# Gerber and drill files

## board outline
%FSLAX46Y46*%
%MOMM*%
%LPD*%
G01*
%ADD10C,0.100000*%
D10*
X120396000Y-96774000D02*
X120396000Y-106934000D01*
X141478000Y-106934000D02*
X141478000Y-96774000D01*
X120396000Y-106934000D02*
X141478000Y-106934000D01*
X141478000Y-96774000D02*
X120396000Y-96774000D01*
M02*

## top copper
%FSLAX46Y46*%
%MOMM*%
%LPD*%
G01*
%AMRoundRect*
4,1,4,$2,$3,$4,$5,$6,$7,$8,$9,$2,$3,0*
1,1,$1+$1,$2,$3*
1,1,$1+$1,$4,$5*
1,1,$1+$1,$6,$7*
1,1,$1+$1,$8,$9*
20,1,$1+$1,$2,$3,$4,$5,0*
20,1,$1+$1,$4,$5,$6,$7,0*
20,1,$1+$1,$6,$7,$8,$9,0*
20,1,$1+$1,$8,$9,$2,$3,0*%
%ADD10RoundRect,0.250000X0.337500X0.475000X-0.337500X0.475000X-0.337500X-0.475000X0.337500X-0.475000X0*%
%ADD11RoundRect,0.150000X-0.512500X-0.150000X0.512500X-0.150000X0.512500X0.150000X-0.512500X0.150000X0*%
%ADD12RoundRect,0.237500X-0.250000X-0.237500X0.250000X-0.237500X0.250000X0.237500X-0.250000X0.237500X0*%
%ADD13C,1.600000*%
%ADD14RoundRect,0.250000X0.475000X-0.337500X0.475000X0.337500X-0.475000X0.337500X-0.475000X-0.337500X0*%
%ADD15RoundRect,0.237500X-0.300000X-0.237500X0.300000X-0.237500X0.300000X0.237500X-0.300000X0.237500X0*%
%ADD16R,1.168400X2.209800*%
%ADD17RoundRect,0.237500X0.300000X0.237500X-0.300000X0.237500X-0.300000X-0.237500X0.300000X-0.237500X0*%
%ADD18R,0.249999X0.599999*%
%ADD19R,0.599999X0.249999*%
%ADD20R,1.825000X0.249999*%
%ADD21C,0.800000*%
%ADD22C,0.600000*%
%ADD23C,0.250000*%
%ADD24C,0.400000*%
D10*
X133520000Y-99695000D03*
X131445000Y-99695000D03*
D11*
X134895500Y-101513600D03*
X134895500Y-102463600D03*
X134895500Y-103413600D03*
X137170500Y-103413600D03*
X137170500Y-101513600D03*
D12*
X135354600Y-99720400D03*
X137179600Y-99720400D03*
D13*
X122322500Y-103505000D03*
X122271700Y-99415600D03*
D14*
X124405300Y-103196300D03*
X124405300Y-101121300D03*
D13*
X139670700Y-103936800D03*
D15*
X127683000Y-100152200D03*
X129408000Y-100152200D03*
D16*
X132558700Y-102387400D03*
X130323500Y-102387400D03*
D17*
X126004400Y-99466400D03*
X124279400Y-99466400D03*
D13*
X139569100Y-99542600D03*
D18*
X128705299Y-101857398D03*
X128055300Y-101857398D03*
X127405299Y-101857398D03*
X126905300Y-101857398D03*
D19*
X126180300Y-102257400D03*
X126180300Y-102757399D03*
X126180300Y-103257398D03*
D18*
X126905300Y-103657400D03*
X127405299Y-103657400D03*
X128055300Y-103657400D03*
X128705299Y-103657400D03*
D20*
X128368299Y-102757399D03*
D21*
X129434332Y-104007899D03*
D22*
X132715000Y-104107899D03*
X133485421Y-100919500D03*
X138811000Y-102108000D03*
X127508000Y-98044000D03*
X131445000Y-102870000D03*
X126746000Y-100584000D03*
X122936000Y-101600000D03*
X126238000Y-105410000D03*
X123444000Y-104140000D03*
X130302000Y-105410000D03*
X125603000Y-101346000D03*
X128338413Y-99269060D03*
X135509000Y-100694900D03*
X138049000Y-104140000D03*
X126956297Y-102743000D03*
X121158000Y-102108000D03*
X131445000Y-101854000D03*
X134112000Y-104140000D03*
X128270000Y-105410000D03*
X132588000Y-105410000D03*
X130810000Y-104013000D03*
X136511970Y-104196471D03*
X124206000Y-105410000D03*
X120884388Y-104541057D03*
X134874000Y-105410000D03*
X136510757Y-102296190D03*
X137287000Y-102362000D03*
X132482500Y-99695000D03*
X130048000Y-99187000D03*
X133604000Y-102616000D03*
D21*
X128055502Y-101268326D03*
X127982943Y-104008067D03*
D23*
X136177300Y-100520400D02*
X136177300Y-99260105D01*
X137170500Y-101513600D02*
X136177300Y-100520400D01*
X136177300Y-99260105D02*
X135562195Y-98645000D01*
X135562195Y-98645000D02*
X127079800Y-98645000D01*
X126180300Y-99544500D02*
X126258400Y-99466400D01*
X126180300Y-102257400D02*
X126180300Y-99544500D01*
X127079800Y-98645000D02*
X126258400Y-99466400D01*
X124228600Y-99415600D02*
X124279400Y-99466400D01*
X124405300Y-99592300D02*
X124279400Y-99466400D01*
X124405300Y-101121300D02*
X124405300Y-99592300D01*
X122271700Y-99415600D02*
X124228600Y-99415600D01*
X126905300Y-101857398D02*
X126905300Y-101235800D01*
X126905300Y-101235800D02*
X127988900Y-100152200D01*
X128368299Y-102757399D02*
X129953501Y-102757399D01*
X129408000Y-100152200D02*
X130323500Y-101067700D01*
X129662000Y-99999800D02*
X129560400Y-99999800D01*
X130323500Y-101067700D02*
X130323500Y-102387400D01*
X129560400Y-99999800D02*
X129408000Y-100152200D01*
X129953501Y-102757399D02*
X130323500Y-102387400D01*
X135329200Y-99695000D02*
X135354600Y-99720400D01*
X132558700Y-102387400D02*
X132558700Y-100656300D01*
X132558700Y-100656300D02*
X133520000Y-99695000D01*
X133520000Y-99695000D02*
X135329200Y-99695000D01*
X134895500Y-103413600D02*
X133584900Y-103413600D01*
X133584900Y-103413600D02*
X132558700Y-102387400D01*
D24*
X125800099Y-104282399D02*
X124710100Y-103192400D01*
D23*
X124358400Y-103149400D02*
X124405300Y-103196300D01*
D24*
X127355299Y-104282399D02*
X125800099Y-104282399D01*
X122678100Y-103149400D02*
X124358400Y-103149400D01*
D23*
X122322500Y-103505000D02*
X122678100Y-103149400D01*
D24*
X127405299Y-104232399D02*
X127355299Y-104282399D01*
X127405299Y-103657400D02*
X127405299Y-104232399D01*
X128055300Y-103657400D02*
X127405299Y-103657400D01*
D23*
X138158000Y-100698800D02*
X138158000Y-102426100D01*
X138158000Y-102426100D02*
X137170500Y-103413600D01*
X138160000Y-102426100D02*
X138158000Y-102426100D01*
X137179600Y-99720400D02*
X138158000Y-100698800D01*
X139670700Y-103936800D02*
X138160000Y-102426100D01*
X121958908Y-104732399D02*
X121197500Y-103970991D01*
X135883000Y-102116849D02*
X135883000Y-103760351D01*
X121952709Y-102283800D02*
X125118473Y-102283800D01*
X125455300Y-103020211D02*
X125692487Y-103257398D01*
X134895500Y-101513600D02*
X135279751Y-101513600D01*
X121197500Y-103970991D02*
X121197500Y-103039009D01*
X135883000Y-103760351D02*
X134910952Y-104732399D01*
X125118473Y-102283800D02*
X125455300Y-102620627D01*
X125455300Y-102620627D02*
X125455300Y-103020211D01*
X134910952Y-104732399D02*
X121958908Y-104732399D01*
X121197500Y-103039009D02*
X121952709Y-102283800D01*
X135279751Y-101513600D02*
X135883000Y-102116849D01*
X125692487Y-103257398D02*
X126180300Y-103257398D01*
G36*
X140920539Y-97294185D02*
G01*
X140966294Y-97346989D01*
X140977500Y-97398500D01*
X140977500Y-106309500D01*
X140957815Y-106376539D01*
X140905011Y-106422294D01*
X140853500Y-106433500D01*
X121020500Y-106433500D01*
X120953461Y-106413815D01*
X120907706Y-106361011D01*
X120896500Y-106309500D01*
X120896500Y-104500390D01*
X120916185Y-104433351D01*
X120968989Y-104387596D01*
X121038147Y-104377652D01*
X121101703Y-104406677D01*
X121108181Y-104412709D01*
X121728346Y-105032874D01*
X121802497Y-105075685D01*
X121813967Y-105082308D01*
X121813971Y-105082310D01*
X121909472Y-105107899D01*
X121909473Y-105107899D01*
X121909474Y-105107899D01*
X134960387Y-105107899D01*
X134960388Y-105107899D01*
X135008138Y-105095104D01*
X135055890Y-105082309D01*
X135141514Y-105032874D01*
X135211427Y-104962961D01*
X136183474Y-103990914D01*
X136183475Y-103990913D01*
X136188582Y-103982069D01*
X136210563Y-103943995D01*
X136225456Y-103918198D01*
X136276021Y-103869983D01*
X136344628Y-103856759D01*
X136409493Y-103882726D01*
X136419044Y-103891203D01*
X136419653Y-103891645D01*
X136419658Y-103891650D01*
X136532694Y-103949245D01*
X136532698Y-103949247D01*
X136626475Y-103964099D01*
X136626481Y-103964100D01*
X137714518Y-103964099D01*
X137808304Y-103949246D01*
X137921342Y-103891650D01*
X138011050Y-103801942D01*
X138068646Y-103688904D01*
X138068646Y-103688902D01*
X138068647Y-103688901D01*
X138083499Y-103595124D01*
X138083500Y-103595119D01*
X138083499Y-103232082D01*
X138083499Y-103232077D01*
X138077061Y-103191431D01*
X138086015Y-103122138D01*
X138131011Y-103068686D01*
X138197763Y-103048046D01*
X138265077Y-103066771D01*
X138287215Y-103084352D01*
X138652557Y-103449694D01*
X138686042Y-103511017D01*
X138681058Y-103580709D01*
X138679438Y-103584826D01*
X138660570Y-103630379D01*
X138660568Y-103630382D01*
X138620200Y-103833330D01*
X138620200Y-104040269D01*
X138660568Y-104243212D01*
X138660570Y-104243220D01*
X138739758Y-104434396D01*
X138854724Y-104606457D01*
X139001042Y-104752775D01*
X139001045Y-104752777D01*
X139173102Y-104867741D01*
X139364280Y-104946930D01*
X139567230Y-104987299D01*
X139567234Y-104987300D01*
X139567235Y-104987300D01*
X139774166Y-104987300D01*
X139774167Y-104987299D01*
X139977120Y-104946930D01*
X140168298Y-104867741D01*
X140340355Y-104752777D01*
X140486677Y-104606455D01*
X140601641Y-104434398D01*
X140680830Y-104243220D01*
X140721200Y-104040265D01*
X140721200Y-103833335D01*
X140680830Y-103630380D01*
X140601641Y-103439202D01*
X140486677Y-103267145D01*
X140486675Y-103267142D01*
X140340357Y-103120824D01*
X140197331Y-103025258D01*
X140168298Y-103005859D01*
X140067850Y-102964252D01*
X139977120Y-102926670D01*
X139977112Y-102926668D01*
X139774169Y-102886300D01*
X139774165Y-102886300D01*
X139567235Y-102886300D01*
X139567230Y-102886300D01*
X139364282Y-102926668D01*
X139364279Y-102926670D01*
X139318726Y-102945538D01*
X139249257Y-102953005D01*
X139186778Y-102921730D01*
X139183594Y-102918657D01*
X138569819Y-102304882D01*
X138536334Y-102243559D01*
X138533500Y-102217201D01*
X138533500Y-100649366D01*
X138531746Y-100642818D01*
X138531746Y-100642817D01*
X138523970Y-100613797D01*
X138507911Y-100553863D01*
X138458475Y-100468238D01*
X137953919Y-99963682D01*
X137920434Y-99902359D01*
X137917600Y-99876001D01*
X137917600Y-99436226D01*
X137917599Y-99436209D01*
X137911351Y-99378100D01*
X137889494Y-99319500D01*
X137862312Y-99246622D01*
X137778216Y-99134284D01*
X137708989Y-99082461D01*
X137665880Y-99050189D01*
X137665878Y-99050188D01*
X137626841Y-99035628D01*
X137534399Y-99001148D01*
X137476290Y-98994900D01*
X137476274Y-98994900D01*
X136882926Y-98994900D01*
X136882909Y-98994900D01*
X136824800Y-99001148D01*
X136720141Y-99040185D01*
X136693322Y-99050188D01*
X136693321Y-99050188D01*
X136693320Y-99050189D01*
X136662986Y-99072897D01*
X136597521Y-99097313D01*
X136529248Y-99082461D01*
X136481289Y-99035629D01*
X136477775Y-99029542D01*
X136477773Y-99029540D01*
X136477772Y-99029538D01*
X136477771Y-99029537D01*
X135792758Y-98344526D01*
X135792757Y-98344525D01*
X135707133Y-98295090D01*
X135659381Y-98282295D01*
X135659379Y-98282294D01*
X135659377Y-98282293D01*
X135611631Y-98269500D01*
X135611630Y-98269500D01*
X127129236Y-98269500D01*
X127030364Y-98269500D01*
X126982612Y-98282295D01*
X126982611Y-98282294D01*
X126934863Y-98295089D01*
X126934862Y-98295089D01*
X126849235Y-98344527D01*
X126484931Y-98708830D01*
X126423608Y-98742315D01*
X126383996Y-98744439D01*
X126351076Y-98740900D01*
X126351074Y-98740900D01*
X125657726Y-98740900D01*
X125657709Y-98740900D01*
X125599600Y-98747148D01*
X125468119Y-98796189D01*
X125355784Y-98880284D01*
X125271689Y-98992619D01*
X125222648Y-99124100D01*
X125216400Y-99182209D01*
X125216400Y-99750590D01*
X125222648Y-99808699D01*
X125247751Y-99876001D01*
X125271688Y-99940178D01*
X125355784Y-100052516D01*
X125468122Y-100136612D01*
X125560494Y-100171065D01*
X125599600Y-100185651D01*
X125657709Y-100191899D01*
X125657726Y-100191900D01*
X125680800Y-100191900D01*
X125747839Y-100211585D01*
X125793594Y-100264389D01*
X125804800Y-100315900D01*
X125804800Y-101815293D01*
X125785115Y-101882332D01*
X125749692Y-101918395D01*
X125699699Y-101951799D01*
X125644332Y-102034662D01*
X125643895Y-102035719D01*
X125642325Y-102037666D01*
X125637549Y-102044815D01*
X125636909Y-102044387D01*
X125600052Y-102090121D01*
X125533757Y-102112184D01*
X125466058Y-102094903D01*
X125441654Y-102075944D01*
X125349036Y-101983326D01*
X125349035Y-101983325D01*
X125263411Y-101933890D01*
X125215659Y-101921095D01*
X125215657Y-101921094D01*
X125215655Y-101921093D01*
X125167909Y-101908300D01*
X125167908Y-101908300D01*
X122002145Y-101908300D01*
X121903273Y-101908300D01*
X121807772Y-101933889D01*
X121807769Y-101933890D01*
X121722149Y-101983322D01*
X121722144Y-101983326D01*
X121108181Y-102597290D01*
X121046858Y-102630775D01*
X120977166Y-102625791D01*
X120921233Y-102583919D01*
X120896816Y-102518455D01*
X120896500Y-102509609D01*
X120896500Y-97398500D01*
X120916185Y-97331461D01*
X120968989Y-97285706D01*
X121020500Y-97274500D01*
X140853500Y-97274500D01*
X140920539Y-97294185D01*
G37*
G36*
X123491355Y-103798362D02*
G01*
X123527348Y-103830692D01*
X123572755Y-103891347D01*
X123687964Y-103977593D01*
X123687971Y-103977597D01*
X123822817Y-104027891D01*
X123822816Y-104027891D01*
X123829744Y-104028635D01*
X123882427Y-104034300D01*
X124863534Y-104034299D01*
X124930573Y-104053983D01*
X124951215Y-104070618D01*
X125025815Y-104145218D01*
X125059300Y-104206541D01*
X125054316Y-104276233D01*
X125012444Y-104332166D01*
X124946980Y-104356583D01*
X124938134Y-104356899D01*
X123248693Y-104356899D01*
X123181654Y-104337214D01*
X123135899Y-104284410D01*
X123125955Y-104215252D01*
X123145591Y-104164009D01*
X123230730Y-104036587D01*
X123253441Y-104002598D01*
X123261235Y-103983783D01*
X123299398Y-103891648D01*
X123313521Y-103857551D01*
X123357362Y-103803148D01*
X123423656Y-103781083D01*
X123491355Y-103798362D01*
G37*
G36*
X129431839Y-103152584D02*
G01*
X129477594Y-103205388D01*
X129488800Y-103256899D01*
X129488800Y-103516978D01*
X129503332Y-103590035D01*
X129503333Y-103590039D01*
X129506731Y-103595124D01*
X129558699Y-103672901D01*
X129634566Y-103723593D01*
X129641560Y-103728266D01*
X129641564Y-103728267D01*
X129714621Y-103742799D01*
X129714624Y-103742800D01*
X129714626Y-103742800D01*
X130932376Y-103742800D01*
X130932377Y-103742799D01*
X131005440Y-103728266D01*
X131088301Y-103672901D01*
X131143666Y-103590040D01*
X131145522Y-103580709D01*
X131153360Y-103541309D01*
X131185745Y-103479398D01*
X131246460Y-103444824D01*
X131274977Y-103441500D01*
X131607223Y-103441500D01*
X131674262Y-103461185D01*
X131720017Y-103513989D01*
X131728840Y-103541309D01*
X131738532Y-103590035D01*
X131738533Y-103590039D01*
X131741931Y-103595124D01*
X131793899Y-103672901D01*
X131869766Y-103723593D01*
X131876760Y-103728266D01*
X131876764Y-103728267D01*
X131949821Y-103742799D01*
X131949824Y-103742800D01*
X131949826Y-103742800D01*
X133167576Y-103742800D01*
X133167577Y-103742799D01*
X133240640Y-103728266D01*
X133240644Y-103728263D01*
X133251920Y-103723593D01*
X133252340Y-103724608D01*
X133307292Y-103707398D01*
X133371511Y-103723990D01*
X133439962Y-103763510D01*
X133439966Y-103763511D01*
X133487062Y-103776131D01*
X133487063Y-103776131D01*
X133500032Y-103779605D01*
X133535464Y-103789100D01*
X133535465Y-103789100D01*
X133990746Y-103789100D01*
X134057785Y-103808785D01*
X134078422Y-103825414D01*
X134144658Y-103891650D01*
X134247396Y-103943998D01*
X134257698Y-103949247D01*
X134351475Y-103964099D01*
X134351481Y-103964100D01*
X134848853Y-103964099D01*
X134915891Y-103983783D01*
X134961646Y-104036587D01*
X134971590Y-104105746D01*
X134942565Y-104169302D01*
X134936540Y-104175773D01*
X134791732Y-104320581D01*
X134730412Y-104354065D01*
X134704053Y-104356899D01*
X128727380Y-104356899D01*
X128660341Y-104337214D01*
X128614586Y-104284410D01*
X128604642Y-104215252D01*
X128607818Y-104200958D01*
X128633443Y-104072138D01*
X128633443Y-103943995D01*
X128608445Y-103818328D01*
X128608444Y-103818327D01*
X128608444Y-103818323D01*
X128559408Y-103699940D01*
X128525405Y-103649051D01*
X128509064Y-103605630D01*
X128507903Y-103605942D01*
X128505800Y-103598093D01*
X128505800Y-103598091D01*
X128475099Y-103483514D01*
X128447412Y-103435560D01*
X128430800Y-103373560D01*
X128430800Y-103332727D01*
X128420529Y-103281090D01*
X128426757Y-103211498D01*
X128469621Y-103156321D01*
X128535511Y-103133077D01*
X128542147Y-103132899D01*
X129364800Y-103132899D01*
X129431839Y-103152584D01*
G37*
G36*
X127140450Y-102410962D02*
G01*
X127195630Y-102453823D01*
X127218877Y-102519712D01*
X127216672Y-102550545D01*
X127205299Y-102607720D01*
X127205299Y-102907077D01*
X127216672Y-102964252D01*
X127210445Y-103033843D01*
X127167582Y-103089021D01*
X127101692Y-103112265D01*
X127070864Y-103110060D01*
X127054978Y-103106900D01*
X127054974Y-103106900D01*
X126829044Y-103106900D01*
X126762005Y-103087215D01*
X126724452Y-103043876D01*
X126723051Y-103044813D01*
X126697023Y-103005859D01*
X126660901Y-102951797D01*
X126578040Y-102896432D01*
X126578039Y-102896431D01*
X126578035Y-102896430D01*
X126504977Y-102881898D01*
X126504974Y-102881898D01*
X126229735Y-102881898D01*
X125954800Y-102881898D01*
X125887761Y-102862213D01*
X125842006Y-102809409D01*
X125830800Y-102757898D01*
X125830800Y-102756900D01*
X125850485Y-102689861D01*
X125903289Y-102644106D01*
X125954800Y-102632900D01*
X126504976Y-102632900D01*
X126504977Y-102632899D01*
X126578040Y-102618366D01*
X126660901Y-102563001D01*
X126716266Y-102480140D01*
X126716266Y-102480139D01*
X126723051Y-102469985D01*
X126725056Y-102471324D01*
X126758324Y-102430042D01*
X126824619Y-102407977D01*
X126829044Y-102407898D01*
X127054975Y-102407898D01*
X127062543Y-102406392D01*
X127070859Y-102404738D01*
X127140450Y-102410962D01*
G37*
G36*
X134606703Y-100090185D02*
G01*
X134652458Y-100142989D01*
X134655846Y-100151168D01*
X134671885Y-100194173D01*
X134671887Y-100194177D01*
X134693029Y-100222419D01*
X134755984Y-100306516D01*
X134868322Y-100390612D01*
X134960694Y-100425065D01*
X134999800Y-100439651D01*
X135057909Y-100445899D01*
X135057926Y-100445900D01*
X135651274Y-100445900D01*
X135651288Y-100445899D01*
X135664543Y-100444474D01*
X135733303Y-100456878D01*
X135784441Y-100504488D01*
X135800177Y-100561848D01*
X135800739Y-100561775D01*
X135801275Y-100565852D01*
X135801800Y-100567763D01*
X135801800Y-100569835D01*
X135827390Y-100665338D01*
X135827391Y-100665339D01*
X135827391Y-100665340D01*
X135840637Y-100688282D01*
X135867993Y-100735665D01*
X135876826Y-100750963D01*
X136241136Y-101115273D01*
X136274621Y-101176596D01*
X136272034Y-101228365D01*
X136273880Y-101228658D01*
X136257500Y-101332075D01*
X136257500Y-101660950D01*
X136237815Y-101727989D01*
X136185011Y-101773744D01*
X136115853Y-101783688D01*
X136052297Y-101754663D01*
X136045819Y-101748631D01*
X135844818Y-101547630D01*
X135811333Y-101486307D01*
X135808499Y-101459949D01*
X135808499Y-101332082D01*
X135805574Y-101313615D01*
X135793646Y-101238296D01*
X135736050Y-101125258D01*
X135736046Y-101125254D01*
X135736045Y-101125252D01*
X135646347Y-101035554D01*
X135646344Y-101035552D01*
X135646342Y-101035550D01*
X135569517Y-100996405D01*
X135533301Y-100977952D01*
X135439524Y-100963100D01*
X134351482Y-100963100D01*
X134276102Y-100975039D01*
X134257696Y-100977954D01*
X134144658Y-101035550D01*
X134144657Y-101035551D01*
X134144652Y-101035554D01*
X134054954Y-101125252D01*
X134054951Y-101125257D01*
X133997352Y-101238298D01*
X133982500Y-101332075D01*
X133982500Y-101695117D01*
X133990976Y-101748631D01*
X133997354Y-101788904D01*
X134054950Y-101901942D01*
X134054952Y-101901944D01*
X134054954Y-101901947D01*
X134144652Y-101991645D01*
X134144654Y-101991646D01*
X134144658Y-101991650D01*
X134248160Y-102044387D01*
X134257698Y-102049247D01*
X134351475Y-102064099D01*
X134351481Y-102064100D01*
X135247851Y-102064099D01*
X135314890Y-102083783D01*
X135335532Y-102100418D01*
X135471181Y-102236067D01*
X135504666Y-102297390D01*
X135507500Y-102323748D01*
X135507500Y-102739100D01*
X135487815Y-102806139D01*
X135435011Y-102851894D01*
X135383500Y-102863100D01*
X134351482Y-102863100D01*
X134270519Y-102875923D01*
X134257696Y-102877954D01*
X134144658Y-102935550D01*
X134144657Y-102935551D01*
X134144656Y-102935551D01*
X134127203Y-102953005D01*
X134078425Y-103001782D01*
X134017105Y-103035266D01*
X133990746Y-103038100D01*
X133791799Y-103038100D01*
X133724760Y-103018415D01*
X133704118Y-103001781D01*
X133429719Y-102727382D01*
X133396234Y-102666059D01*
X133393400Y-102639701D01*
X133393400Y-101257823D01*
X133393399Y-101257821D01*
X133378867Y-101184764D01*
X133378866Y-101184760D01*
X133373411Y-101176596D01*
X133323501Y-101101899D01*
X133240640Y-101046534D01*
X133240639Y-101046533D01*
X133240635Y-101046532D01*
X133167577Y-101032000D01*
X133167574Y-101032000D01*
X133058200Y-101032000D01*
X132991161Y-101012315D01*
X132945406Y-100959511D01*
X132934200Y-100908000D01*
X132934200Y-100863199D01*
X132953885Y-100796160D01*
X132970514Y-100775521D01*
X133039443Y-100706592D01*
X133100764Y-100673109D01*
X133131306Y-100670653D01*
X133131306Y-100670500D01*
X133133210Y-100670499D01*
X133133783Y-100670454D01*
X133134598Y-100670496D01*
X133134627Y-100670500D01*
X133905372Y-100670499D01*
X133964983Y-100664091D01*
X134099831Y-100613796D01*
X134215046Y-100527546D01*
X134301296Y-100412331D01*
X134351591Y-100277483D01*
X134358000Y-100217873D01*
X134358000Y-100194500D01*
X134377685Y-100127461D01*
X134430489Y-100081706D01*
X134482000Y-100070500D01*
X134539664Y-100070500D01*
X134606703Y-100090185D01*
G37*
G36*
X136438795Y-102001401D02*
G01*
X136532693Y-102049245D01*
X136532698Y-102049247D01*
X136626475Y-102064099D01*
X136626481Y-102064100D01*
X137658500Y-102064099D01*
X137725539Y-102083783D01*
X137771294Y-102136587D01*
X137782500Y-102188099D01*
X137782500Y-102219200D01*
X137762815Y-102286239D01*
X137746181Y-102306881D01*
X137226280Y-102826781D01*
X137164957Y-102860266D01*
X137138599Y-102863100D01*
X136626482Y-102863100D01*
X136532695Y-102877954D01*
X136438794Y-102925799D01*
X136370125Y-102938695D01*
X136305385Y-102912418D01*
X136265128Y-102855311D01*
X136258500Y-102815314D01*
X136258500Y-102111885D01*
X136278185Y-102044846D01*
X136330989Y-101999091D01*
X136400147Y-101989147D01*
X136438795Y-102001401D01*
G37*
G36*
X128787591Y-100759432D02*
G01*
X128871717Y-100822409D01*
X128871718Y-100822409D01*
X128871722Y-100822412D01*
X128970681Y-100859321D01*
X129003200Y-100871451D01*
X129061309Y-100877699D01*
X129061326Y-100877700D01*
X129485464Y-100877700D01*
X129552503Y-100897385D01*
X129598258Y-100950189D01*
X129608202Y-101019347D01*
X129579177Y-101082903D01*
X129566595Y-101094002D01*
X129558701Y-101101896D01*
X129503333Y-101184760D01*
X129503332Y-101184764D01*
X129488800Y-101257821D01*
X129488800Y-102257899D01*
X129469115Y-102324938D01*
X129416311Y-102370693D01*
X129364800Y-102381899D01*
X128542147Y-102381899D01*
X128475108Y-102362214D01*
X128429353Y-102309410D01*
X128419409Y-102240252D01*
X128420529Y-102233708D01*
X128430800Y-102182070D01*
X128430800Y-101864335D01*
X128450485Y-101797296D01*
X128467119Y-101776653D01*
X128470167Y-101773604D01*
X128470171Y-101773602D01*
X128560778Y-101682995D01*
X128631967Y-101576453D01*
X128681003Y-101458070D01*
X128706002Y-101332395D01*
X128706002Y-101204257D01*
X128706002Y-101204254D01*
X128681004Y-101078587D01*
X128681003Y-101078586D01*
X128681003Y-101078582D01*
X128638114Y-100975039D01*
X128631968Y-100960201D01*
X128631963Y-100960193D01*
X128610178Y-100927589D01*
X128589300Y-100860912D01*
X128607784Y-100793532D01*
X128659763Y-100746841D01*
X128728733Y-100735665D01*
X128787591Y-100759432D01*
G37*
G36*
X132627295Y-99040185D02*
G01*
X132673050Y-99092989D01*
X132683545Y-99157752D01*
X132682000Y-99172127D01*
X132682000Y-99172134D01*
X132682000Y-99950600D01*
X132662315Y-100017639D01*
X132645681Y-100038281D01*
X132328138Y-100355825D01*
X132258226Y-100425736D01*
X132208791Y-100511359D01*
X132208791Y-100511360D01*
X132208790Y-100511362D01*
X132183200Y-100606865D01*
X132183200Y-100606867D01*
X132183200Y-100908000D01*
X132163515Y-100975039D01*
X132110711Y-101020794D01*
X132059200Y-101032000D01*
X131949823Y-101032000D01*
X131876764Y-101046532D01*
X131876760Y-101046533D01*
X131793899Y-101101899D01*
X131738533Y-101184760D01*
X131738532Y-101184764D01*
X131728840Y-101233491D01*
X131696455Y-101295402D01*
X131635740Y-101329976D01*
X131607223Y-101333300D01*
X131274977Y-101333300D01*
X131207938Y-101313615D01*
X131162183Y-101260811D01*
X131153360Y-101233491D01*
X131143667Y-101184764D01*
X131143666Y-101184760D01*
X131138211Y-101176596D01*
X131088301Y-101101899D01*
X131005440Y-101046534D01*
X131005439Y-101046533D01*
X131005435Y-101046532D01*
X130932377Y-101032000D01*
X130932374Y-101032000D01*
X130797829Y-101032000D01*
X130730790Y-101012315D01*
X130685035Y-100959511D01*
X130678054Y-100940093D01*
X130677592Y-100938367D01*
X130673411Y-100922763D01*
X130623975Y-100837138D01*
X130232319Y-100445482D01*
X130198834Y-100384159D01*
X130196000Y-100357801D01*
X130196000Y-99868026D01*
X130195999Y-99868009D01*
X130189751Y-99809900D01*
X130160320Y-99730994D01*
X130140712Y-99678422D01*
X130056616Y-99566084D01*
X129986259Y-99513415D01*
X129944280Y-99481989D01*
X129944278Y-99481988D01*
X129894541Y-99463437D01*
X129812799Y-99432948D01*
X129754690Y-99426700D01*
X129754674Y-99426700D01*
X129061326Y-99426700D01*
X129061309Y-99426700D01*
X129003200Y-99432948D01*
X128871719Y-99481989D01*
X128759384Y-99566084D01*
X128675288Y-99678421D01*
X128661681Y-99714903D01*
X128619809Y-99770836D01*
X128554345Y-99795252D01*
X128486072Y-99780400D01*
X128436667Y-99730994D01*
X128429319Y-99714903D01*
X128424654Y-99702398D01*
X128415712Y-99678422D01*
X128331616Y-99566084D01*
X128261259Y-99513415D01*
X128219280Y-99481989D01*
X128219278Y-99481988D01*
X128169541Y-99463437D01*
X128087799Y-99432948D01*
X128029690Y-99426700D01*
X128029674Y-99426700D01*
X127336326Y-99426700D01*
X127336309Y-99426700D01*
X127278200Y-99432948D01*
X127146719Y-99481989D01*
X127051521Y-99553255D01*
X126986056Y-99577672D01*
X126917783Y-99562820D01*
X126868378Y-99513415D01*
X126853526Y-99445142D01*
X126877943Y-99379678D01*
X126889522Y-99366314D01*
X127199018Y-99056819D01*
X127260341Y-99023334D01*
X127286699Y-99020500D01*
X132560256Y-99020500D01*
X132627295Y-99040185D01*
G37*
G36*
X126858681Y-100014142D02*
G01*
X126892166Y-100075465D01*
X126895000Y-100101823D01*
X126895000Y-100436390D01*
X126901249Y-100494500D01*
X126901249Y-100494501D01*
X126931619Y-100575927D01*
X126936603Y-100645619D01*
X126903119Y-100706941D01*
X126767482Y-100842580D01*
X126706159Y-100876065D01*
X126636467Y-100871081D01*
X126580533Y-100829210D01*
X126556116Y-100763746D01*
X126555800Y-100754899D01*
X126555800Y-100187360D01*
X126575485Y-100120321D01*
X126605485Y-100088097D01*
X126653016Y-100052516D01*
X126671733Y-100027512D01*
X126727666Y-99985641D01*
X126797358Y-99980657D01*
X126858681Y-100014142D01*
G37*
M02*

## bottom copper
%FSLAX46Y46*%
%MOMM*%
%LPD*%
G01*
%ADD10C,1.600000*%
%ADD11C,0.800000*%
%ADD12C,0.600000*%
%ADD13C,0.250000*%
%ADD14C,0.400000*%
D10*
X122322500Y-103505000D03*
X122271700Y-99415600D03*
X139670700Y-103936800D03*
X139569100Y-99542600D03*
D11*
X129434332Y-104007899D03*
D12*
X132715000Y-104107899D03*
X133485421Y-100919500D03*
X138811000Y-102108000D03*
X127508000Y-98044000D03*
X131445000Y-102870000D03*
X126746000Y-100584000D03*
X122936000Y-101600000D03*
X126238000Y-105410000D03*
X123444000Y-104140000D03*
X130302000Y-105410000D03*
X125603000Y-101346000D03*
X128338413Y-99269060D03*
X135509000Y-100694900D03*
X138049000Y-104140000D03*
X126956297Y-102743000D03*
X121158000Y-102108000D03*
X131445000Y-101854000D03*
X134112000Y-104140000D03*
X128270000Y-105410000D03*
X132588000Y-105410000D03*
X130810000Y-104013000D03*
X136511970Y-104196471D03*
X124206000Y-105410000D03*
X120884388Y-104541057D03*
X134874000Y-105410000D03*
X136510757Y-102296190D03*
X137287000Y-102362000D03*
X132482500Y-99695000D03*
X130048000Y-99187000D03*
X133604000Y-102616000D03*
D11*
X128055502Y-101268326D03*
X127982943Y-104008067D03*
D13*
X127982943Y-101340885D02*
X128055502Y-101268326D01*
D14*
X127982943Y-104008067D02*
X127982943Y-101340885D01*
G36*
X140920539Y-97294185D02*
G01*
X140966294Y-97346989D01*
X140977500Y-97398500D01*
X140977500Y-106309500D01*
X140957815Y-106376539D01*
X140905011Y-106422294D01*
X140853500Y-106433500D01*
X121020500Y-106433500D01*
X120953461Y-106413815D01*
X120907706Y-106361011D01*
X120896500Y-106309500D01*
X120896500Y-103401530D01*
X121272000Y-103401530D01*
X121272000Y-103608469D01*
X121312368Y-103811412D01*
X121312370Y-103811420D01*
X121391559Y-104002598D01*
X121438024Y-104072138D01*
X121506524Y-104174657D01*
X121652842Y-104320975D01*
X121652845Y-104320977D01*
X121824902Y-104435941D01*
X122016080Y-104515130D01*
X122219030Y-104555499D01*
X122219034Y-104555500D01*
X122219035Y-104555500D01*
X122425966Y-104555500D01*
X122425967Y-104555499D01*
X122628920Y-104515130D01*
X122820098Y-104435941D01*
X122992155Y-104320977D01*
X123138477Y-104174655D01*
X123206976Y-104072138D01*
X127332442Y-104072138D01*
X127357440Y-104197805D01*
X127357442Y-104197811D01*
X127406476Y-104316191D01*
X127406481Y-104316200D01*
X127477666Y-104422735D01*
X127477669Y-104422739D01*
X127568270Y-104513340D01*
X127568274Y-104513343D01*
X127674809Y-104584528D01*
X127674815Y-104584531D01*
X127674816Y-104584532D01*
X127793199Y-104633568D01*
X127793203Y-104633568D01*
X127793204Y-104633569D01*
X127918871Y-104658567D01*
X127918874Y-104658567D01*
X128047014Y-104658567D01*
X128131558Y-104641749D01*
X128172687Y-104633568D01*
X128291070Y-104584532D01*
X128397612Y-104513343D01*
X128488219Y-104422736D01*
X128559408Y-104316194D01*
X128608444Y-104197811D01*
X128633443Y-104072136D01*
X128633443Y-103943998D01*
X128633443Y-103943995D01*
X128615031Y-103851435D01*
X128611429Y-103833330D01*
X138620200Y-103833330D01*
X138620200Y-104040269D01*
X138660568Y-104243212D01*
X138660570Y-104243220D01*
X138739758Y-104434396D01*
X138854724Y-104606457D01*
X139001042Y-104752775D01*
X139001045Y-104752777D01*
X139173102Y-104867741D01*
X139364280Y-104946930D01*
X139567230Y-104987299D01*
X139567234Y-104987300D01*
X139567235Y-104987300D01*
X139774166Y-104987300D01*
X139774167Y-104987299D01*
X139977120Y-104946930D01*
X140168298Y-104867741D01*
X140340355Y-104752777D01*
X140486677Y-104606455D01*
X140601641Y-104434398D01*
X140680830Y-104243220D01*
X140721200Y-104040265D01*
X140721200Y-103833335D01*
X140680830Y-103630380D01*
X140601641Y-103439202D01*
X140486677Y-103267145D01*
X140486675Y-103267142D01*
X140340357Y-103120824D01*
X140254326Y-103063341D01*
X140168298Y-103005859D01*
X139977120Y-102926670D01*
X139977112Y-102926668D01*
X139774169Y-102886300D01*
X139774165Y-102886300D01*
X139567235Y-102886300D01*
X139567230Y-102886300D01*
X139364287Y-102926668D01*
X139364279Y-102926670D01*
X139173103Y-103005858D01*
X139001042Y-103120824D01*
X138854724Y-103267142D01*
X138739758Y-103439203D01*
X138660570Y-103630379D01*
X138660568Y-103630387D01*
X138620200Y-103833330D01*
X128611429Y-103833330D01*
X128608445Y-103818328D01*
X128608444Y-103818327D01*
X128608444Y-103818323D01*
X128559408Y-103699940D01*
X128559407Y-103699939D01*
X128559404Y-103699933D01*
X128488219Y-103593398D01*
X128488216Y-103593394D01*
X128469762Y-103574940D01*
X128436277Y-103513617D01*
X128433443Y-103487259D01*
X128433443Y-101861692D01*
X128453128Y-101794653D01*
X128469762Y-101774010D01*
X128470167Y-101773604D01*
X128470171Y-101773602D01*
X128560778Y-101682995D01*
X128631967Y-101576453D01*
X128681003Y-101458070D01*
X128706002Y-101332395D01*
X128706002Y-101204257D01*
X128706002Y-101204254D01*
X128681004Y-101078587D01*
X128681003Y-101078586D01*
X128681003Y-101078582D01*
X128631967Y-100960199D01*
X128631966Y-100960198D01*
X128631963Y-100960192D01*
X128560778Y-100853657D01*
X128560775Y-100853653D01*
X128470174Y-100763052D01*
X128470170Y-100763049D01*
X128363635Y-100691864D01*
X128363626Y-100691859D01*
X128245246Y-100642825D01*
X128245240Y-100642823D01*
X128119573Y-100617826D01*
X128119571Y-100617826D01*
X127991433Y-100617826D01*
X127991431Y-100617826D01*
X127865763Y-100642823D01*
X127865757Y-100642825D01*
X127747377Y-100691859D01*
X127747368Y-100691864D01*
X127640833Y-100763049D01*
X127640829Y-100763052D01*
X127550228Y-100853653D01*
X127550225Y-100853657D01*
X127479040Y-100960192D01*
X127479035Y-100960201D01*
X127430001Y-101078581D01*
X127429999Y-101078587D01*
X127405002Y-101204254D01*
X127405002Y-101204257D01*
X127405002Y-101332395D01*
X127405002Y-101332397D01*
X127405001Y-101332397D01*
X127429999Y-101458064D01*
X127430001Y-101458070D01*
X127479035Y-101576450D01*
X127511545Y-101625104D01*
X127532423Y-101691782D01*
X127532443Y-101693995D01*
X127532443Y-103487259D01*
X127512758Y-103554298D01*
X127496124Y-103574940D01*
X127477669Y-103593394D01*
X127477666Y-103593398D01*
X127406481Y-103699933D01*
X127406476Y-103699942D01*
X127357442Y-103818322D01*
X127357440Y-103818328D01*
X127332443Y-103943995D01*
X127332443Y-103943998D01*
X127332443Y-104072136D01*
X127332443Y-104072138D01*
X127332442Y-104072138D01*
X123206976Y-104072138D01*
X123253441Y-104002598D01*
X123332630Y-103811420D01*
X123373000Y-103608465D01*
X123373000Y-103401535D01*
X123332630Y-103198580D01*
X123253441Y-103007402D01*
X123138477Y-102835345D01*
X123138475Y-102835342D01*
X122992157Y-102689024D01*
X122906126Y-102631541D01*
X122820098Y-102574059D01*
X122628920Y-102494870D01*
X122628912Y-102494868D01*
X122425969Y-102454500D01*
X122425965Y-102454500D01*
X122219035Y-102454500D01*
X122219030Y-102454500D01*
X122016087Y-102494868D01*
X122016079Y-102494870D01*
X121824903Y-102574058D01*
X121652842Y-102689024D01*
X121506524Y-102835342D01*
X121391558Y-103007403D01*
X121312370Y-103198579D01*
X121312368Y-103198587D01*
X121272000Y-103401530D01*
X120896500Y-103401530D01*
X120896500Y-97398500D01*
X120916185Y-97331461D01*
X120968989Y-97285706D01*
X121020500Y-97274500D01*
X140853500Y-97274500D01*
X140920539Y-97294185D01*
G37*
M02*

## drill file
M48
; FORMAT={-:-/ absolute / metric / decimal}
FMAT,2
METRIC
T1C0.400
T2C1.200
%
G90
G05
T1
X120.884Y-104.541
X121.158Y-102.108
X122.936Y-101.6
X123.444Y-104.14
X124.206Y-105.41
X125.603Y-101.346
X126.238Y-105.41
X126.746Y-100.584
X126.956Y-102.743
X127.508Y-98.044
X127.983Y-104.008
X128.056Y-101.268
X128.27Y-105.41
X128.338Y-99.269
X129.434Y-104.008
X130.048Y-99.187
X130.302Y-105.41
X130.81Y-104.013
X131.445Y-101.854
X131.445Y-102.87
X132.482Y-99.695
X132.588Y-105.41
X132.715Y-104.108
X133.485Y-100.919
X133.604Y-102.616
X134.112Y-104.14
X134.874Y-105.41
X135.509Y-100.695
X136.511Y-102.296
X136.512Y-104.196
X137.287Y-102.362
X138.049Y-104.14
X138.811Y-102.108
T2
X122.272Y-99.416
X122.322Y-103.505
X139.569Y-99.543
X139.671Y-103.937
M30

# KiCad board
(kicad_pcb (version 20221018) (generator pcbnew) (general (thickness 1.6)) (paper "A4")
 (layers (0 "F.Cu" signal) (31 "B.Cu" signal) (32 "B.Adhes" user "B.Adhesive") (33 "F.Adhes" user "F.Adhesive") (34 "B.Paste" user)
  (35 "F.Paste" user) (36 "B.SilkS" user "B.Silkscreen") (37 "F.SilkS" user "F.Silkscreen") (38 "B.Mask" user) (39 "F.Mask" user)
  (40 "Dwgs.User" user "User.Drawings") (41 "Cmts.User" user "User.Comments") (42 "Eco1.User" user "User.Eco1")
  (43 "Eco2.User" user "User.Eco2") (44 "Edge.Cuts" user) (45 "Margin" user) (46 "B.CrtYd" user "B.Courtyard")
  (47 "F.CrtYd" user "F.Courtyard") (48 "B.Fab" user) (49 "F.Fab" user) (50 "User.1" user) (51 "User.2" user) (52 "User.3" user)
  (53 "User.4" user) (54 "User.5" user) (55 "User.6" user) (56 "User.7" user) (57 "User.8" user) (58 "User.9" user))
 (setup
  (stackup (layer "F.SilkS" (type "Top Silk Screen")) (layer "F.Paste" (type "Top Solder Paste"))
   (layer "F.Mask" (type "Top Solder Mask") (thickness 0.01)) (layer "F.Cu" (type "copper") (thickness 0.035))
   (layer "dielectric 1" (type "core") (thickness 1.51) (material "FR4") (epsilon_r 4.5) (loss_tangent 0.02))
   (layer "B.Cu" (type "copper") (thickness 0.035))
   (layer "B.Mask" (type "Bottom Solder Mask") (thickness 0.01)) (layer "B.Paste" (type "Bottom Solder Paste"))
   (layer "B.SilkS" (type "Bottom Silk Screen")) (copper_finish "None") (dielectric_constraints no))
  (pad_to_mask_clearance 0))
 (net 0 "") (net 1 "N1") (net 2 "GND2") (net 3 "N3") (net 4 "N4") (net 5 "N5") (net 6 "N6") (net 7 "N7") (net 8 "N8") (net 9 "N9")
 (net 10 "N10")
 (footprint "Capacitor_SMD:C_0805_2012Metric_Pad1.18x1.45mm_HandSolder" (layer "F.Cu") (at 132.4825 99.695 180)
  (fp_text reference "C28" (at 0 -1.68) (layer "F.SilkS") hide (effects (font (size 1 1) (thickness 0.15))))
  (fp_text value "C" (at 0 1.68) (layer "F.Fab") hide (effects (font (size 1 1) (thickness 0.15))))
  (pad "1" smd roundrect (at -1.0375 0 180) (size 1.175 1.45) (layers "F.Cu" "F.Paste" "F.Mask") (roundrect_rratio 0.2127659574)
   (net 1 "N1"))
  (pad "2" smd roundrect (at 1.0375 0 180) (size 1.175 1.45) (layers "F.Cu" "F.Paste" "F.Mask") (roundrect_rratio 0.2127659574)
   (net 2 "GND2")))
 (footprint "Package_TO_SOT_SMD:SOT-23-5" (layer "F.Cu") (at 136.033 102.4636)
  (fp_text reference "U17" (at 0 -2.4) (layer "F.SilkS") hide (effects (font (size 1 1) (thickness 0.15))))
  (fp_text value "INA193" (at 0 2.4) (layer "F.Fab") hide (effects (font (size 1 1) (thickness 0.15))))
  (pad "1" smd roundrect (at -1.1375 -0.95) (size 1.325 0.6) (layers "F.Cu" "F.Paste" "F.Mask") (roundrect_rratio 0.25) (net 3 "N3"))
  (pad "2" smd roundrect (at -1.1375 0) (size 1.325 0.6) (layers "F.Cu" "F.Paste" "F.Mask") (roundrect_rratio 0.25) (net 2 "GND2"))
  (pad "3" smd roundrect (at -1.1375 0.95) (size 1.325 0.6) (layers "F.Cu" "F.Paste" "F.Mask") (roundrect_rratio 0.25) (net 1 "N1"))
  (pad "4" smd roundrect (at 1.1375 0.95) (size 1.325 0.6) (layers "F.Cu" "F.Paste" "F.Mask") (roundrect_rratio 0.25) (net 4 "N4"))
  (pad "5" smd roundrect (at 1.1375 -0.95) (size 1.325 0.6) (layers "F.Cu" "F.Paste" "F.Mask") (roundrect_rratio 0.25) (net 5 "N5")))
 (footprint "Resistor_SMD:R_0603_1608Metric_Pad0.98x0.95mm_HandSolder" (layer "F.Cu") (at 136.2671 99.7204)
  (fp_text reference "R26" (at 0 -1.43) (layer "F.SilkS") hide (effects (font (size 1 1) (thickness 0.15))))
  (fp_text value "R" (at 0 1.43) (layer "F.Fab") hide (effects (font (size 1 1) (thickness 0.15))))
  (pad "1" smd roundrect (at -0.9125 0) (size 0.975 0.95) (layers "F.Cu" "F.Paste" "F.Mask") (roundrect_rratio 0.25) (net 1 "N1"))
  (pad "2" smd roundrect (at 0.9125 0) (size 0.975 0.95) (layers "F.Cu" "F.Paste" "F.Mask") (roundrect_rratio 0.25) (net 4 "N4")))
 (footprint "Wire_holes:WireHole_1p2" (layer "F.Cu") (at 122.3225 103.505)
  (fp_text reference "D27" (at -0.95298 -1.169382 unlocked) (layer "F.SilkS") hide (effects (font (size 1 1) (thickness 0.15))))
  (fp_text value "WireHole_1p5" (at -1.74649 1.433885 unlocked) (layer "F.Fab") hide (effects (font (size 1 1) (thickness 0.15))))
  (pad "1" thru_hole circle (at 0 0) (size 1.6 1.6) (drill 1.2) (layers "*.Cu" "*.Mask") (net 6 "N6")))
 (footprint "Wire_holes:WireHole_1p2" (layer "F.Cu") (at 122.2717 99.4156)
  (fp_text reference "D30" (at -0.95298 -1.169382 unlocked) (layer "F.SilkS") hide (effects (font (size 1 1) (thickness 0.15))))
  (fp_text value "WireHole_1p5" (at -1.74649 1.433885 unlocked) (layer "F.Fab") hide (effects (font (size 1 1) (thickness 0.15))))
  (pad "1" thru_hole circle (at 0 0) (size 1.6 1.6) (drill 1.2) (layers "*.Cu" "*.Mask") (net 2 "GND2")))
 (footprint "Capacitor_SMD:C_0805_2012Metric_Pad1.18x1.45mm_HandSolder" (layer "F.Cu") (at 124.4053 102.1588 90)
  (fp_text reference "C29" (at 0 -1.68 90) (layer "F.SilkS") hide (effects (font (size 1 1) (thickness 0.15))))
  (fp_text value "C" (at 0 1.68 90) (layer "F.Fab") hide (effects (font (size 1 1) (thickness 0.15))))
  (pad "1" smd roundrect (at -1.0375 0 90) (size 1.175 1.45) (layers "F.Cu" "F.Paste" "F.Mask") (roundrect_rratio 0.2127659574) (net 6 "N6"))
  (pad "2" smd roundrect (at 1.0375 0 90) (size 1.175 1.45) (layers "F.Cu" "F.Paste" "F.Mask") (roundrect_rratio 0.2127659574)
   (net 2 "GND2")))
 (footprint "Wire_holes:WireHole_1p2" (layer "F.Cu") (at 139.6707 103.9368)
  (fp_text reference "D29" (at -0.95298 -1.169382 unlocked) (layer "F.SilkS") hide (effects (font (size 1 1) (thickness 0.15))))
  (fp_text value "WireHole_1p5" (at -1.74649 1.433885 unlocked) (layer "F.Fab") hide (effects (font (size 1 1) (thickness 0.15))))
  (pad "1" thru_hole circle (at 0 0) (size 1.6 1.6) (drill 1.2) (layers "*.Cu" "*.Mask") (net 4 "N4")))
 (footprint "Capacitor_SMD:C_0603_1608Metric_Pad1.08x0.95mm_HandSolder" (layer "F.Cu") (at 128.5455 100.1522)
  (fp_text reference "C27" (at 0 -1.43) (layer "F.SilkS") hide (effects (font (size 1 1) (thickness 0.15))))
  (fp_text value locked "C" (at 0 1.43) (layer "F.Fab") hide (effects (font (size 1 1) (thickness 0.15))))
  (pad "1" smd roundrect (at -0.8625 0) (size 1.075 0.95) (layers "F.Cu" "F.Paste" "F.Mask") (roundrect_rratio 0.25) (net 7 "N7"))
  (pad "2" smd roundrect (at 0.8625 0) (size 1.075 0.95) (layers "F.Cu" "F.Paste" "F.Mask") (roundrect_rratio 0.25) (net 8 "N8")))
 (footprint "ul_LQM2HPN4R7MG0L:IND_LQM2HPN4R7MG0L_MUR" (layer "F.Cu") (at 131.4411 102.3874 180)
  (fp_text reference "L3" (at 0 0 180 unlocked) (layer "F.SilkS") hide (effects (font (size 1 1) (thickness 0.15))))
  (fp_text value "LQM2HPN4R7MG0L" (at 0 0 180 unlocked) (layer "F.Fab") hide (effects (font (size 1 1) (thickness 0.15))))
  (pad "1" smd rect (at -1.1176 0 180) (size 1.1684 2.2098) (layers "F.Cu" "F.Paste" "F.Mask") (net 1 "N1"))
  (pad "2" smd rect (at 1.1176 0 180) (size 1.1684 2.2098) (layers "F.Cu" "F.Paste" "F.Mask") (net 8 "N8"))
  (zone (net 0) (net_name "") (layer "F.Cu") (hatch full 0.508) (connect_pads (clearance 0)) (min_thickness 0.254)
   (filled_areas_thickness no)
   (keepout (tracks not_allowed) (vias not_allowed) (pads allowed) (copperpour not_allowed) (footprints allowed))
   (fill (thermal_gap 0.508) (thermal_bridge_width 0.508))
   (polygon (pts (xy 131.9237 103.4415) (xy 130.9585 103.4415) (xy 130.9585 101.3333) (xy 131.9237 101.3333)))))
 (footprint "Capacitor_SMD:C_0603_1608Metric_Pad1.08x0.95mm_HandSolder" (layer "F.Cu") (at 125.1419 99.4664 180)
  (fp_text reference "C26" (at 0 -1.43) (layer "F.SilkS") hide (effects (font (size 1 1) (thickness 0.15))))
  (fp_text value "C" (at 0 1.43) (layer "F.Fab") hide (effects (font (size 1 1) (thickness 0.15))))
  (pad "1" smd roundrect (at -0.8625 0 180) (size 1.075 0.95) (layers "F.Cu" "F.Paste" "F.Mask") (roundrect_rratio 0.25) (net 5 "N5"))
  (pad "2" smd roundrect (at 0.8625 0 180) (size 1.075 0.95) (layers "F.Cu" "F.Paste" "F.Mask") (roundrect_rratio 0.25) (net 2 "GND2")))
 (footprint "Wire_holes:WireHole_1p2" (layer "F.Cu") (at 139.5691 99.5426)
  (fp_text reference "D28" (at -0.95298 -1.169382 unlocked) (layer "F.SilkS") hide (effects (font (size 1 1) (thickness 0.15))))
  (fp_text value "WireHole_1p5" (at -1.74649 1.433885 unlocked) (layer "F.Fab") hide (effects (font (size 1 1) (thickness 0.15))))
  (pad "1" thru_hole circle (at 0 0) (size 1.6 1.6) (drill 1.2) (layers "*.Cu" "*.Mask") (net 2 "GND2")))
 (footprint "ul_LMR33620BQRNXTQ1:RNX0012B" (layer "F.Cu") (at 127.5803 102.757399 -90)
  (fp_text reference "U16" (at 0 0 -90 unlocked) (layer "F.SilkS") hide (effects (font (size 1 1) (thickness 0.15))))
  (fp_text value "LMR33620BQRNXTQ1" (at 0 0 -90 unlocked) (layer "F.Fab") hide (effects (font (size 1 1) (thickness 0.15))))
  (pad "1" smd rect (at -0.900001 -1.124999 270) (size 0.599999 0.249999) (layers "F.Cu" "F.Paste" "F.Mask") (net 2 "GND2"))
  (pad "2" smd rect (at -0.900001 -0.475 270) (size 0.599999 0.249999) (layers "F.Cu" "F.Paste" "F.Mask") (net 6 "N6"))
  (pad "3" smd rect (at -0.900001 0.175001 270) (size 0.599999 0.249999) (layers "F.Cu" "F.Paste" "F.Mask") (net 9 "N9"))
  (pad "4" smd rect (at -0.900001 0.675 270) (size 0.599999 0.249999) (layers "F.Cu" "F.Paste" "F.Mask") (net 7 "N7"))
  (pad "5" smd rect (at -0.499999 1.4) (size 0.599999 0.249999) (layers "F.Cu" "F.Paste" "F.Mask") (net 5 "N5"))
  (pad "6" smd rect (at 0 1.4) (size 0.599999 0.249999) (layers "F.Cu" "F.Paste" "F.Mask") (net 2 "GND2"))
  (pad "7" smd rect (at 0.499999 1.4) (size 0.599999 0.249999) (layers "F.Cu" "F.Paste" "F.Mask") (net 3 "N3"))
  (pad "8" smd rect (at 0.900001 0.675 270) (size 0.599999 0.249999) (layers "F.Cu" "F.Paste" "F.Mask") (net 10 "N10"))
  (pad "9" smd rect (at 0.900001 0.175001 270) (size 0.599999 0.249999) (layers "F.Cu" "F.Paste" "F.Mask") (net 6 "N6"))
  (pad "10" smd rect (at 0.900001 -0.475 270) (size 0.599999 0.249999) (layers "F.Cu" "F.Paste" "F.Mask") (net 6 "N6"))
  (pad "11" smd rect (at 0.900001 -1.124999 270) (size 0.599999 0.249999) (layers "F.Cu" "F.Paste" "F.Mask") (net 2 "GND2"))
  (pad "12" smd rect (at 0 -0.787999) (size 1.825 0.249999) (layers "F.Cu" "F.Mask") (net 8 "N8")))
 (gr_line (start 120.396 96.774) (end 120.396 106.934) (stroke (width 0.1) (type default)) (layer "Edge.Cuts"))
 (gr_line (start 141.478 106.934) (end 141.478 96.774) (stroke (width 0.1) (type default)) (layer "Edge.Cuts"))
 (gr_line (start 120.396 106.934) (end 141.478 106.934) (stroke (width 0.1) (type default)) (layer "Edge.Cuts"))
 (gr_line (start 141.478 96.774) (end 120.396 96.774) (stroke (width 0.1) (type default)) (layer "Edge.Cuts"))
 (segment (start 136.1773 100.5204) (end 136.1773 99.260105) (width 0.25) (layer "F.Cu") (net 5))
 (segment (start 137.1705 101.5136) (end 136.1773 100.5204) (width 0.25) (layer "F.Cu") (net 5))
 (segment (start 136.1773 99.260105) (end 135.562195 98.645) (width 0.25) (layer "F.Cu") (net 5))
 (segment (start 135.562195 98.645) (end 127.0798 98.645) (width 0.25) (layer "F.Cu") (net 5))
 (segment (start 126.1803 99.5445) (end 126.2584 99.4664) (width 0.25) (layer "F.Cu") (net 5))
 (segment (start 126.1803 102.2574) (end 126.1803 99.5445) (width 0.25) (layer "F.Cu") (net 5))
 (segment (start 127.0798 98.645) (end 126.2584 99.4664) (width 0.25) (layer "F.Cu") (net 5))
 (segment (start 124.2286 99.4156) (end 124.2794 99.4664) (width 0.25) (layer "F.Cu") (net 2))
 (segment (start 124.4053 99.5923) (end 124.2794 99.4664) (width 0.25) (layer "F.Cu") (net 2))
 (segment (start 124.4053 101.1213) (end 124.4053 99.5923) (width 0.25) (layer "F.Cu") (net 2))
 (segment (start 122.2717 99.4156) (end 124.2286 99.4156) (width 0.25) (layer "F.Cu") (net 2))
 (via (at 129.434332 104.007899) (size 0.8) (drill 0.4) (layers "F.Cu" "B.Cu") (free) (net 2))
 (via (at 132.715 104.107899) (size 0.6) (drill 0.4) (layers "F.Cu" "B.Cu") (free) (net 2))
 (via (at 133.485421 100.9195) (size 0.6) (drill 0.4) (layers "F.Cu" "B.Cu") (free) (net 2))
 (via (at 138.811 102.108) (size 0.6) (drill 0.4) (layers "F.Cu" "B.Cu") (free) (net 2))
 (via (at 127.508 98.044) (size 0.6) (drill 0.4) (layers "F.Cu" "B.Cu") (free) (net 2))
 (via (at 131.445 102.87) (size 0.6) (drill 0.4) (layers "F.Cu" "B.Cu") (free) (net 2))
 (via (at 126.746 100.584) (size 0.6) (drill 0.4) (layers "F.Cu" "B.Cu") (free) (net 2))
 (via (at 122.936 101.6) (size 0.6) (drill 0.4) (layers "F.Cu" "B.Cu") (free) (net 2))
 (via (at 126.238 105.41) (size 0.6) (drill 0.4) (layers "F.Cu" "B.Cu") (free) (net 2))
 (via (at 123.444 104.14) (size 0.6) (drill 0.4) (layers "F.Cu" "B.Cu") (free) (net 2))
 (via (at 130.302 105.41) (size 0.6) (drill 0.4) (layers "F.Cu" "B.Cu") (free) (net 2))
 (via (at 125.603 101.346) (size 0.6) (drill 0.4) (layers "F.Cu" "B.Cu") (free) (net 2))
 (via (at 128.338413 99.26906) (size 0.6) (drill 0.4) (layers "F.Cu" "B.Cu") (free) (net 2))
 (via (at 135.509 100.6949) (size 0.6) (drill 0.4) (layers "F.Cu" "B.Cu") (free) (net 2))
 (via (at 138.049 104.14) (size 0.6) (drill 0.4) (layers "F.Cu" "B.Cu") (free) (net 2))
 (via (at 126.956297 102.743) (size 0.6) (drill 0.4) (layers "F.Cu" "B.Cu") (free) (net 2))
 (via (at 121.158 102.108) (size 0.6) (drill 0.4) (layers "F.Cu" "B.Cu") (free) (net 2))
 (via (at 131.445 101.854) (size 0.6) (drill 0.4) (layers "F.Cu" "B.Cu") (free) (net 2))
 (via (at 134.112 104.14) (size 0.6) (drill 0.4) (layers "F.Cu" "B.Cu") (free) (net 2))
 (via (at 128.27 105.41) (size 0.6) (drill 0.4) (layers "F.Cu" "B.Cu") (free) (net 2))
 (via (at 132.588 105.41) (size 0.6) (drill 0.4) (layers "F.Cu" "B.Cu") (free) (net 2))
 (via (at 130.81 104.013) (size 0.6) (drill 0.4) (layers "F.Cu" "B.Cu") (free) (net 2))
 (via (at 136.51197 104.196471) (size 0.6) (drill 0.4) (layers "F.Cu" "B.Cu") (free) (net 2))
 (via (at 124.206 105.41) (size 0.6) (drill 0.4) (layers "F.Cu" "B.Cu") (free) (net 2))
 (via (at 120.884388 104.541057) (size 0.6) (drill 0.4) (layers "F.Cu" "B.Cu") (free) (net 2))
 (via (at 134.874 105.41) (size 0.6) (drill 0.4) (layers "F.Cu" "B.Cu") (free) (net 2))
 (via (at 136.510757 102.29619) (size 0.6) (drill 0.4) (layers "F.Cu" "B.Cu") (free) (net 2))
 (via (at 137.287 102.362) (size 0.6) (drill 0.4) (layers "F.Cu" "B.Cu") (free) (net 2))
 (via (at 132.4825 99.695) (size 0.6) (drill 0.4) (layers "F.Cu" "B.Cu") (free) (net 2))
 (via (at 130.048 99.187) (size 0.6) (drill 0.4) (layers "F.Cu" "B.Cu") (free) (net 2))
 (via (at 133.604 102.616) (size 0.6) (drill 0.4) (layers "F.Cu" "B.Cu") (free) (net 2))
 (segment (start 126.9053 101.857398) (end 126.9053 101.2358) (width 0.25) (layer "F.Cu") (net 7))
 (segment (start 126.9053 101.2358) (end 127.9889 100.1522) (width 0.25) (layer "F.Cu") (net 7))
 (segment (start 128.368299 102.757399) (end 129.953501 102.757399) (width 0.25) (layer "F.Cu") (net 8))
 (segment (start 129.408 100.1522) (end 130.3235 101.0677) (width 0.25) (layer "F.Cu") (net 8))
 (segment (start 129.662 99.9998) (end 129.5604 99.9998) (width 0.25) (layer "F.Cu") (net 8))
 (segment (start 130.3235 101.0677) (end 130.3235 102.3874) (width 0.25) (layer "F.Cu") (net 8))
 (segment (start 129.5604 99.9998) (end 129.408 100.1522) (width 0.25) (layer "F.Cu") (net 8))
 (segment (start 129.953501 102.757399) (end 130.3235 102.3874) (width 0.25) (layer "F.Cu") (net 8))
 (segment (start 135.3292 99.695) (end 135.3546 99.7204) (width 0.25) (layer "F.Cu") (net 1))
 (segment (start 132.5587 102.3874) (end 132.5587 100.6563) (width 0.25) (layer "F.Cu") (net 1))
 (segment (start 132.5587 100.6563) (end 133.52 99.695) (width 0.25) (layer "F.Cu") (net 1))
 (segment (start 133.52 99.695) (end 135.3292 99.695) (width 0.25) (layer "F.Cu") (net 1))
 (segment (start 134.8955 103.4136) (end 133.5849 103.4136) (width 0.25) (layer "F.Cu") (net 1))
 (segment (start 133.5849 103.4136) (end 132.5587 102.3874) (width 0.25) (layer "F.Cu") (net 1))
 (segment (start 125.800099 104.282399) (end 124.7101 103.1924) (width 0.4) (layer "F.Cu") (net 6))
 (segment (start 124.3584 103.1494) (end 124.4053 103.1963) (width 0.25) (layer "F.Cu") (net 6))
 (segment (start 127.355299 104.282399) (end 125.800099 104.282399) (width 0.4) (layer "F.Cu") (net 6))
 (segment (start 122.6781 103.1494) (end 124.3584 103.1494) (width 0.4) (layer "F.Cu") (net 6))
 (segment (start 122.3225 103.505) (end 122.6781 103.1494) (width 0.25) (layer "F.Cu") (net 6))
 (segment (start 127.405299 104.232399) (end 127.355299 104.282399) (width 0.4) (layer "F.Cu") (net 6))
 (segment (start 127.405299 103.6574) (end 127.405299 104.232399) (width 0.4) (layer "F.Cu") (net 6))
 (segment (start 128.0553 103.6574) (end 127.405299 103.6574) (width 0.4) (layer "F.Cu") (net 6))
 (via (at 128.055502 101.268326) (size 0.8) (drill 0.4) (layers "F.Cu" "B.Cu") (free) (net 6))
 (via (at 127.982943 104.008067) (size 0.8) (drill 0.4) (layers "F.Cu" "B.Cu") (free) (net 6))
 (segment (start 127.982943 101.340885) (end 128.055502 101.268326) (width 0.25) (layer "B.Cu") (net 6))
 (segment (start 127.982943 104.008067) (end 127.982943 101.340885) (width 0.4) (layer "B.Cu") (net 6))
 (segment (start 138.158 100.6988) (end 138.158 102.4261) (width 0.25) (layer "F.Cu") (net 4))
 (segment (start 138.158 102.4261) (end 137.1705 103.4136) (width 0.25) (layer "F.Cu") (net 4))
 (segment (start 138.16 102.4261) (end 138.158 102.4261) (width 0.25) (layer "F.Cu") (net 4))
 (segment (start 137.1796 99.7204) (end 138.158 100.6988) (width 0.25) (layer "F.Cu") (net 4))
 (segment (start 139.6707 103.9368) (end 138.16 102.4261) (width 0.25) (layer "F.Cu") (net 4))
 (segment (start 121.958908 104.732399) (end 121.1975 103.970991) (width 0.25) (layer "F.Cu") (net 3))
 (segment (start 135.883 102.116849) (end 135.883 103.760351) (width 0.25) (layer "F.Cu") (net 3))
 (segment (start 121.952709 102.2838) (end 125.118473 102.2838) (width 0.25) (layer "F.Cu") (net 3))
 (segment (start 125.4553 103.020211) (end 125.692487 103.257398) (width 0.25) (layer "F.Cu") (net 3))
 (segment (start 134.8955 101.5136) (end 135.279751 101.5136) (width 0.25) (layer "F.Cu") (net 3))
 (segment (start 121.1975 103.970991) (end 121.1975 103.039009) (width 0.25) (layer "F.Cu") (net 3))
 (segment (start 135.883 103.760351) (end 134.910952 104.732399) (width 0.25) (layer "F.Cu") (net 3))
 (segment (start 125.118473 102.2838) (end 125.4553 102.620627) (width 0.25) (layer "F.Cu") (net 3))
 (segment (start 125.4553 102.620627) (end 125.4553 103.020211) (width 0.25) (layer "F.Cu") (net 3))
 (segment (start 134.910952 104.732399) (end 121.958908 104.732399) (width 0.25) (layer "F.Cu") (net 3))
 (segment (start 121.1975 103.039009) (end 121.952709 102.2838) (width 0.25) (layer "F.Cu") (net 3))
 (segment (start 135.279751 101.5136) (end 135.883 102.116849) (width 0.25) (layer "F.Cu") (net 3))
 (segment (start 125.692487 103.257398) (end 126.1803 103.257398) (width 0.25) (layer "F.Cu") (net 3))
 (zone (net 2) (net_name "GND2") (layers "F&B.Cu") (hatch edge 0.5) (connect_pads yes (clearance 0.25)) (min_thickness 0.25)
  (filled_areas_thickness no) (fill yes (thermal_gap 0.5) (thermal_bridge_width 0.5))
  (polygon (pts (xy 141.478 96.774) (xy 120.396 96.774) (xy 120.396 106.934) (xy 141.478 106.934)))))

